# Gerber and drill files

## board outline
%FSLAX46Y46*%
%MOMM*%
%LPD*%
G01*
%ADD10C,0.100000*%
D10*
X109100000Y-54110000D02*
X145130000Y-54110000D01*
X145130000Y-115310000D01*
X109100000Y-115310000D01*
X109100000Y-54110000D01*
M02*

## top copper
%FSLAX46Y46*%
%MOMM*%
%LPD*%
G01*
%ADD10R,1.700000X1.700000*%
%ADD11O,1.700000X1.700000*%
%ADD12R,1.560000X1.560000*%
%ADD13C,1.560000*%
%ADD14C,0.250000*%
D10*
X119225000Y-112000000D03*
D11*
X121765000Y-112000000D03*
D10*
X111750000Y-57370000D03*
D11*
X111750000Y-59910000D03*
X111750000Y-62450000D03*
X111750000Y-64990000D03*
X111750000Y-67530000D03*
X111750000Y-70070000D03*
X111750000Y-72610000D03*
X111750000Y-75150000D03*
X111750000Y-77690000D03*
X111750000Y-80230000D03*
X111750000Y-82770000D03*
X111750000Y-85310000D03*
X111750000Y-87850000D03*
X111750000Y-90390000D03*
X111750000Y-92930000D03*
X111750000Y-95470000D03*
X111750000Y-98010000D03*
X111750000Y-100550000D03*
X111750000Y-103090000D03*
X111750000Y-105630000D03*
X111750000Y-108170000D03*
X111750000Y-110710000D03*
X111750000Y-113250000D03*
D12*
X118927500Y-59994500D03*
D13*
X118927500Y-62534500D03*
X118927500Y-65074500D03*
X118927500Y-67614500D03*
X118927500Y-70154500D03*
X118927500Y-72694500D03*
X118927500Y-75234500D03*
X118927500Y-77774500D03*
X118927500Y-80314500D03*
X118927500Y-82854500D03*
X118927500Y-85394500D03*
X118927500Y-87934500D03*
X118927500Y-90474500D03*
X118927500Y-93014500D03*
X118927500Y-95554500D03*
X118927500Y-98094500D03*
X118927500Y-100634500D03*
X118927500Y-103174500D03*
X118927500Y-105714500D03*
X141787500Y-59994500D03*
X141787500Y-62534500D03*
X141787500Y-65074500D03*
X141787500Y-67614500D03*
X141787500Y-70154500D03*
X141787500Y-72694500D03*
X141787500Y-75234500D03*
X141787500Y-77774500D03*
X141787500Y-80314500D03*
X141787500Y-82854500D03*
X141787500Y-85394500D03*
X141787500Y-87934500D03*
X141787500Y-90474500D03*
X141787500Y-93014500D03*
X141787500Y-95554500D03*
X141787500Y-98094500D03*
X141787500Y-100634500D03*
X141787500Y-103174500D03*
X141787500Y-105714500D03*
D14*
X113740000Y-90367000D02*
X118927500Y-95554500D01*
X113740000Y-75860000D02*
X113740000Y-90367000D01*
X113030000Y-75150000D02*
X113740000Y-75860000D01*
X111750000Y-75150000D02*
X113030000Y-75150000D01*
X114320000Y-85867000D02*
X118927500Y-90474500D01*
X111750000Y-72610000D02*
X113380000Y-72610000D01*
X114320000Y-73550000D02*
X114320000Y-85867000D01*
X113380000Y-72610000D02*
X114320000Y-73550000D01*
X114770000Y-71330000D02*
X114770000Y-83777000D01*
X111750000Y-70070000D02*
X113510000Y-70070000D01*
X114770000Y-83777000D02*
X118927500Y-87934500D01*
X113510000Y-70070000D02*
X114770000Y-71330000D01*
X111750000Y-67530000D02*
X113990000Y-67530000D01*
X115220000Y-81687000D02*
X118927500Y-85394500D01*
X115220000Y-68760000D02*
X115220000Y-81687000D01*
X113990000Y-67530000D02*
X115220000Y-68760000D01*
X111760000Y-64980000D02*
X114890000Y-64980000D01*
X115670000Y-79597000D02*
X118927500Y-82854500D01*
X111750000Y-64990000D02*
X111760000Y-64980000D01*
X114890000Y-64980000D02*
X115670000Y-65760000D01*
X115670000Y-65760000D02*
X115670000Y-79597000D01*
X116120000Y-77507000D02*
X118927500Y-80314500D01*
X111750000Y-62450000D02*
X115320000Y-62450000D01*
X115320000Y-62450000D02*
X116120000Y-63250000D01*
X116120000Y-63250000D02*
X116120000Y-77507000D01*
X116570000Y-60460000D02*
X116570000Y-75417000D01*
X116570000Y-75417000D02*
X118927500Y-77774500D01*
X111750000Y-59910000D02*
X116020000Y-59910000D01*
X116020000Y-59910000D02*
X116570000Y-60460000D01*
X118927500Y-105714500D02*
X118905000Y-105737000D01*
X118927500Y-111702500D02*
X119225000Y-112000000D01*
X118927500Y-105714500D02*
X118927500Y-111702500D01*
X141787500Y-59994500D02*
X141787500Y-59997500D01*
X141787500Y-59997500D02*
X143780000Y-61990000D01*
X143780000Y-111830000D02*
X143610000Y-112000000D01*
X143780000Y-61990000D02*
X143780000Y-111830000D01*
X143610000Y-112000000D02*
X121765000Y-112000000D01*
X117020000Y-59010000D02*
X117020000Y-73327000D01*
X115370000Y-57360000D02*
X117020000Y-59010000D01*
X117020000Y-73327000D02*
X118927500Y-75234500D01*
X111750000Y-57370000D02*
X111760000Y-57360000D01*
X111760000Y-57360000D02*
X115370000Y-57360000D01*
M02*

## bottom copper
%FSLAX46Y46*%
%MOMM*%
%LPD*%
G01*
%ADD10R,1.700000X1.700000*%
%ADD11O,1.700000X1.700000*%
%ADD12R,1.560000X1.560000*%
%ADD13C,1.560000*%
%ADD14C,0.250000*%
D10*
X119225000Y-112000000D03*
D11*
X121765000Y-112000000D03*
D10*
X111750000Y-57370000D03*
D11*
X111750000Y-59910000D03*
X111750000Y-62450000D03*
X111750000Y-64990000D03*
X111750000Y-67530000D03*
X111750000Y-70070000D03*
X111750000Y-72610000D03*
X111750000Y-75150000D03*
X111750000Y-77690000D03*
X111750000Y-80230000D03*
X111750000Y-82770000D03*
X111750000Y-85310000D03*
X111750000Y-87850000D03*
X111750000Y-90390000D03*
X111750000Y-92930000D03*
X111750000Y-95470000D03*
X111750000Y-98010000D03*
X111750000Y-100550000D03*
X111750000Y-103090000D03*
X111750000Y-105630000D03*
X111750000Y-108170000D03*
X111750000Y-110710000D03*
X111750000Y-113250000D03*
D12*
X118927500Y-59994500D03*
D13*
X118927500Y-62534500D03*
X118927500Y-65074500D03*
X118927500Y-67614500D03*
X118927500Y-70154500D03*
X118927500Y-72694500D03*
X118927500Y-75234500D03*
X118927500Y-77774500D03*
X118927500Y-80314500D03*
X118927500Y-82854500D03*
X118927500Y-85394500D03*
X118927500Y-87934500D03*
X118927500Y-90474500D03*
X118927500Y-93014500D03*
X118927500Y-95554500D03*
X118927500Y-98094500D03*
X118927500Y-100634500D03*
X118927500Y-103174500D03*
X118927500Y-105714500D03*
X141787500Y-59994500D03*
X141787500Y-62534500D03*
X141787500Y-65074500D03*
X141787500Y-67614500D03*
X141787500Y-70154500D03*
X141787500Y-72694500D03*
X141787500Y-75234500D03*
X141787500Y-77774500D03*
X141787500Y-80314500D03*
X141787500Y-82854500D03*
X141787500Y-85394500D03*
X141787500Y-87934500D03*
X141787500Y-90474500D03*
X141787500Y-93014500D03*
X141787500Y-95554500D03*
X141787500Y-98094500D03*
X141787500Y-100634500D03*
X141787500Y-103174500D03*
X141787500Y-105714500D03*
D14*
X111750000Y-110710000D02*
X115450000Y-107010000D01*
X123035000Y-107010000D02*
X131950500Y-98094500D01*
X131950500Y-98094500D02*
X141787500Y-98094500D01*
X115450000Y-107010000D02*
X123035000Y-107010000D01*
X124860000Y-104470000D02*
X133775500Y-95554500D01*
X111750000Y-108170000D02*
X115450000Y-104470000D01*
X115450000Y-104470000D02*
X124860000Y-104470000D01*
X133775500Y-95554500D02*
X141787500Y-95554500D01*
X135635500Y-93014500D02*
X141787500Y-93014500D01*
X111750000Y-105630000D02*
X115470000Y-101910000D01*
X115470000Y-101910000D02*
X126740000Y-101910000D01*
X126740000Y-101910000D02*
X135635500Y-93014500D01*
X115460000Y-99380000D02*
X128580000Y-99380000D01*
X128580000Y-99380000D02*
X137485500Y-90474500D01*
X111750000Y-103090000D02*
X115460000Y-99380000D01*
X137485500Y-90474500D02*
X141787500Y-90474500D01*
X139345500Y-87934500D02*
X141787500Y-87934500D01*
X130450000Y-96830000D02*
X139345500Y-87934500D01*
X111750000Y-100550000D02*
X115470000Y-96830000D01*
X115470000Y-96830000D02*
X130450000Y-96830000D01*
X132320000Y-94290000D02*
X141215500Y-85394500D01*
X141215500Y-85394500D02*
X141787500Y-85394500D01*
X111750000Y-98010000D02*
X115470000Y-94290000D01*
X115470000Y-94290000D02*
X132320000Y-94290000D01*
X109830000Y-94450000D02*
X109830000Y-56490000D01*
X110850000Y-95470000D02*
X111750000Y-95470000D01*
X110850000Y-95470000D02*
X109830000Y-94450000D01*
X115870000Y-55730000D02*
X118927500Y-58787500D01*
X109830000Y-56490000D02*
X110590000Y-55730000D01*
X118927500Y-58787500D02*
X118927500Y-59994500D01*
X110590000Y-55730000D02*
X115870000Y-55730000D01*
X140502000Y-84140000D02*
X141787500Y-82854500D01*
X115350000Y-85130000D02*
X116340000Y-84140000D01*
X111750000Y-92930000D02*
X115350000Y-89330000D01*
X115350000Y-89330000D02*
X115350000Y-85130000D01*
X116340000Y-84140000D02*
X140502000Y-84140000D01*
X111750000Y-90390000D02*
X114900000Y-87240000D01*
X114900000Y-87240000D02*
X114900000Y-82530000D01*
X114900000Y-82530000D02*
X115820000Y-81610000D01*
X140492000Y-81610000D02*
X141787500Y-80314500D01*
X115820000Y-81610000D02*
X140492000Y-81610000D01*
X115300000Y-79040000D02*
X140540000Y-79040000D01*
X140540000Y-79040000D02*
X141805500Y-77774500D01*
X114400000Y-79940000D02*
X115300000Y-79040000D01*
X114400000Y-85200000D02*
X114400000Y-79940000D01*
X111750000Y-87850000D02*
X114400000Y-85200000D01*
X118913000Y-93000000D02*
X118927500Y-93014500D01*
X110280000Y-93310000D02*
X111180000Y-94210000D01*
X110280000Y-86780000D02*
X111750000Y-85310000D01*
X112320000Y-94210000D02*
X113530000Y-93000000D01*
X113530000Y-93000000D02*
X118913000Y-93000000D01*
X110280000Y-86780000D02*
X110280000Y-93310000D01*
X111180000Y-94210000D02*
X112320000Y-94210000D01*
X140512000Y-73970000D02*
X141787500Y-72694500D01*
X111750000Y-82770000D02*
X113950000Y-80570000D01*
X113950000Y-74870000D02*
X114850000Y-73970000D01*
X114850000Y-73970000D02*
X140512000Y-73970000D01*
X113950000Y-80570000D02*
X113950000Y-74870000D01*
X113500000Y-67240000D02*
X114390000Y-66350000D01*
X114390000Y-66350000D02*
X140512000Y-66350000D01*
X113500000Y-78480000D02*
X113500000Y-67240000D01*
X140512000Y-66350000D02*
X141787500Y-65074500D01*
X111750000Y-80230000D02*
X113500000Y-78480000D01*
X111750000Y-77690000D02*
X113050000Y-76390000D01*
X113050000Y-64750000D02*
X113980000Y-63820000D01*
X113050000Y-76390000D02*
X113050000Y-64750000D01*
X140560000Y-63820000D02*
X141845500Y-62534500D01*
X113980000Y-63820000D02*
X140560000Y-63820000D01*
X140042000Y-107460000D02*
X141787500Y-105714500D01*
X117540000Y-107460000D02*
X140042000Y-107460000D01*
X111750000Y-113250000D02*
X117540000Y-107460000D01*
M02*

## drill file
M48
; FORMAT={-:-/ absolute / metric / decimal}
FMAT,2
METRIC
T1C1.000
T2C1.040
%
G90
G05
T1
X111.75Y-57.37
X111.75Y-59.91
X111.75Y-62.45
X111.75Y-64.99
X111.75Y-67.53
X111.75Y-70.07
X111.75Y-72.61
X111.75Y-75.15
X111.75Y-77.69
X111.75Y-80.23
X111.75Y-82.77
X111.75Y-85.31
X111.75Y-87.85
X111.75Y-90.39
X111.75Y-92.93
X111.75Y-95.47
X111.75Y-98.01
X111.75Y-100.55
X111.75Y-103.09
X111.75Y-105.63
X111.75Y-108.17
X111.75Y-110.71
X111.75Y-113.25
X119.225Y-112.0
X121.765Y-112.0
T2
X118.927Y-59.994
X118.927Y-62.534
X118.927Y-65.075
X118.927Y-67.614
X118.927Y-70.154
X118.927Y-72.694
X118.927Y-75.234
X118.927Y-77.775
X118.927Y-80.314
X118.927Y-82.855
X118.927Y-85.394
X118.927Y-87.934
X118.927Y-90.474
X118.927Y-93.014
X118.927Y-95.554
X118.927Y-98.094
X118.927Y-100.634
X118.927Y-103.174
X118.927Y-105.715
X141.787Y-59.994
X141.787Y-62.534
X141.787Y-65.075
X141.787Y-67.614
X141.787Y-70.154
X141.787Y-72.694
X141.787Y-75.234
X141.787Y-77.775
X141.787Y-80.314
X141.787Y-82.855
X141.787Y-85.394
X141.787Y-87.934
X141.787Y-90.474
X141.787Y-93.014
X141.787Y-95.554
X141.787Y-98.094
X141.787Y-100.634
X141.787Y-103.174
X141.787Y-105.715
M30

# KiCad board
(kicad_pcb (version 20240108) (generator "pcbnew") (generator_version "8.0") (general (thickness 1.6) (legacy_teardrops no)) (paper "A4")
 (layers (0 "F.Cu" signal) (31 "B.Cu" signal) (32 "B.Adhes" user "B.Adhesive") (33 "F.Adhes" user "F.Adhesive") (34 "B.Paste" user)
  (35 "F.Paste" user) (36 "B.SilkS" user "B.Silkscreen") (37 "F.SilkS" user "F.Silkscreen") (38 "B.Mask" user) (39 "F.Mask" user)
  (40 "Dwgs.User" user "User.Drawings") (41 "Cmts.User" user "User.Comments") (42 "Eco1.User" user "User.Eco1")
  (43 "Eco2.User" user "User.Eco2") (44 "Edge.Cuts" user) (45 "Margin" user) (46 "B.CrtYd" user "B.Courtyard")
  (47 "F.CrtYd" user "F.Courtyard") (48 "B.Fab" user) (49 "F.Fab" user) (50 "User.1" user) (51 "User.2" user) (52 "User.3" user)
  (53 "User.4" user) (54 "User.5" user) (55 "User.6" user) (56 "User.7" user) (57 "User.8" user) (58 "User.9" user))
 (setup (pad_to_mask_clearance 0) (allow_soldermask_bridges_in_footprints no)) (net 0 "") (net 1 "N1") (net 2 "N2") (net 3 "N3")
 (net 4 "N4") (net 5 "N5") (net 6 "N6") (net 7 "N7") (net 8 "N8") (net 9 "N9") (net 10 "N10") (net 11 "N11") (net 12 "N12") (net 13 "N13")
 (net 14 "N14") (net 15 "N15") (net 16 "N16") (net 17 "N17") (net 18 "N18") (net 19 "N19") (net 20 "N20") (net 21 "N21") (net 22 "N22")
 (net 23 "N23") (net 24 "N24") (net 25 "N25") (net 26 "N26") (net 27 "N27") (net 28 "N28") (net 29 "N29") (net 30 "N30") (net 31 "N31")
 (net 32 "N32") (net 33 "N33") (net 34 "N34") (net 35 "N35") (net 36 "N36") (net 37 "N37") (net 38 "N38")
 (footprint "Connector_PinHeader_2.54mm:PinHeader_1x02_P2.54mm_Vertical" (layer "F.Cu") (at 119.225 112 90)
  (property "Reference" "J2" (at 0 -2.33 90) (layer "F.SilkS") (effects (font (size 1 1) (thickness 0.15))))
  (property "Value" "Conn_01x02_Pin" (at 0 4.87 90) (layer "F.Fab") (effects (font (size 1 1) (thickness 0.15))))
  (pad "1" thru_hole rect (at 0 0 90) (size 1.7 1.7) (drill 1) (layers "*.Cu" "*.Mask") (remove_unused_layers no) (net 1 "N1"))
  (pad "2" thru_hole oval (at 0 2.54 90) (size 1.7 1.7) (drill 1) (layers "*.Cu" "*.Mask") (remove_unused_layers no) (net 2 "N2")))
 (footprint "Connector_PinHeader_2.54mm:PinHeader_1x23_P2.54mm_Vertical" (layer "F.Cu") (at 111.75 57.37)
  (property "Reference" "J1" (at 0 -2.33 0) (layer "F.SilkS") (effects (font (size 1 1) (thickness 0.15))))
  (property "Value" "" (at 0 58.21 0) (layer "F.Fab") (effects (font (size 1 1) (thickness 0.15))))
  (pad "1" thru_hole rect (at 0 0) (size 1.7 1.7) (drill 1) (layers "*.Cu" "*.Mask") (remove_unused_layers no) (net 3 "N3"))
  (pad "2" thru_hole oval (at 0 2.54) (size 1.7 1.7) (drill 1) (layers "*.Cu" "*.Mask") (remove_unused_layers no) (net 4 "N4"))
  (pad "3" thru_hole oval (at 0 5.08) (size 1.7 1.7) (drill 1) (layers "*.Cu" "*.Mask") (remove_unused_layers no) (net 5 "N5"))
  (pad "4" thru_hole oval (at 0 7.62) (size 1.7 1.7) (drill 1) (layers "*.Cu" "*.Mask") (remove_unused_layers no) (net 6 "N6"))
  (pad "5" thru_hole oval (at 0 10.16) (size 1.7 1.7) (drill 1) (layers "*.Cu" "*.Mask") (remove_unused_layers no) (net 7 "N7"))
  (pad "6" thru_hole oval (at 0 12.7) (size 1.7 1.7) (drill 1) (layers "*.Cu" "*.Mask") (remove_unused_layers no) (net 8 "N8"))
  (pad "7" thru_hole oval (at 0 15.24) (size 1.7 1.7) (drill 1) (layers "*.Cu" "*.Mask") (remove_unused_layers no) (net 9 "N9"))
  (pad "8" thru_hole oval (at 0 17.78) (size 1.7 1.7) (drill 1) (layers "*.Cu" "*.Mask") (remove_unused_layers no) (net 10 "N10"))
  (pad "9" thru_hole oval (at 0 20.32) (size 1.7 1.7) (drill 1) (layers "*.Cu" "*.Mask") (remove_unused_layers no) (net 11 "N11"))
  (pad "10" thru_hole oval (at 0 22.86) (size 1.7 1.7) (drill 1) (layers "*.Cu" "*.Mask") (remove_unused_layers no) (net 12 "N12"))
  (pad "11" thru_hole oval (at 0 25.4) (size 1.7 1.7) (drill 1) (layers "*.Cu" "*.Mask") (remove_unused_layers no) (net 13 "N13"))
  (pad "12" thru_hole oval (at 0 27.94) (size 1.7 1.7) (drill 1) (layers "*.Cu" "*.Mask") (remove_unused_layers no) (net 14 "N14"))
  (pad "13" thru_hole oval (at 0 30.48) (size 1.7 1.7) (drill 1) (layers "*.Cu" "*.Mask") (remove_unused_layers no) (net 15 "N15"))
  (pad "14" thru_hole oval (at 0 33.02) (size 1.7 1.7) (drill 1) (layers "*.Cu" "*.Mask") (remove_unused_layers no) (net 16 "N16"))
  (pad "15" thru_hole oval (at 0 35.56) (size 1.7 1.7) (drill 1) (layers "*.Cu" "*.Mask") (remove_unused_layers no) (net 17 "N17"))
  (pad "16" thru_hole oval (at 0 38.1) (size 1.7 1.7) (drill 1) (layers "*.Cu" "*.Mask") (remove_unused_layers no) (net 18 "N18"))
  (pad "17" thru_hole oval (at 0 40.64) (size 1.7 1.7) (drill 1) (layers "*.Cu" "*.Mask") (remove_unused_layers no) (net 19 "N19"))
  (pad "18" thru_hole oval (at 0 43.18) (size 1.7 1.7) (drill 1) (layers "*.Cu" "*.Mask") (remove_unused_layers no) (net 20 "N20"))
  (pad "19" thru_hole oval (at 0 45.72) (size 1.7 1.7) (drill 1) (layers "*.Cu" "*.Mask") (remove_unused_layers no) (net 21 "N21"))
  (pad "20" thru_hole oval (at 0 48.26) (size 1.7 1.7) (drill 1) (layers "*.Cu" "*.Mask") (remove_unused_layers no) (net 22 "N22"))
  (pad "21" thru_hole oval (at 0 50.8) (size 1.7 1.7) (drill 1) (layers "*.Cu" "*.Mask") (remove_unused_layers no) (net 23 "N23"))
  (pad "22" thru_hole oval (at 0 53.34) (size 1.7 1.7) (drill 1) (layers "*.Cu" "*.Mask") (remove_unused_layers no) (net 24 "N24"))
  (pad "23" thru_hole oval (at 0 55.88) (size 1.7 1.7) (drill 1) (layers "*.Cu" "*.Mask") (remove_unused_layers no) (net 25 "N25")))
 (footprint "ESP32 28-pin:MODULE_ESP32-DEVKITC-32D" (layer "F.Cu") (at 131.6275 79.7545)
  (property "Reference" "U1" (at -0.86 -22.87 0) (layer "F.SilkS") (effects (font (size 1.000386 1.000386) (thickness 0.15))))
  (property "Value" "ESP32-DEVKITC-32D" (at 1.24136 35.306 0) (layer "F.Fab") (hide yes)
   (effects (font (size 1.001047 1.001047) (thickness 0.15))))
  (pad "J2-1" thru_hole rect (at -12.7 -19.76) (size 1.56 1.56) (drill 1.04) (layers "*.Cu" "*.Mask") (remove_unused_layers no)
   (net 18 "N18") (solder_mask_margin 0.102))
  (pad "J2-2" thru_hole circle (at -12.7 -17.22) (size 1.56 1.56) (drill 1.04) (layers "*.Cu" "*.Mask") (remove_unused_layers no)
   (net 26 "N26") (solder_mask_margin 0.102))
  (pad "J2-3" thru_hole circle (at -12.7 -14.68) (size 1.56 1.56) (drill 1.04) (layers "*.Cu" "*.Mask") (remove_unused_layers no)
   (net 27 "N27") (solder_mask_margin 0.102))
  (pad "J2-4" thru_hole circle (at -12.7 -12.14) (size 1.56 1.56) (drill 1.04) (layers "*.Cu" "*.Mask") (remove_unused_layers no)
   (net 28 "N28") (solder_mask_margin 0.102))
  (pad "J2-5" thru_hole circle (at -12.7 -9.6) (size 1.56 1.56) (drill 1.04) (layers "*.Cu" "*.Mask") (remove_unused_layers no)
   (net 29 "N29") (solder_mask_margin 0.102))
  (pad "J2-6" thru_hole circle (at -12.7 -7.06) (size 1.56 1.56) (drill 1.04) (layers "*.Cu" "*.Mask") (remove_unused_layers no)
   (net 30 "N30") (solder_mask_margin 0.102))
  (pad "J2-7" thru_hole circle (at -12.7 -4.52) (size 1.56 1.56) (drill 1.04) (layers "*.Cu" "*.Mask") (remove_unused_layers no)
   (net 3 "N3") (solder_mask_margin 0.102))
  (pad "J2-8" thru_hole circle (at -12.7 -1.98) (size 1.56 1.56) (drill 1.04) (layers "*.Cu" "*.Mask") (remove_unused_layers no)
   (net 4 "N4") (solder_mask_margin 0.102))
  (pad "J2-9" thru_hole circle (at -12.7 0.56) (size 1.56 1.56) (drill 1.04) (layers "*.Cu" "*.Mask") (remove_unused_layers no) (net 5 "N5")
   (solder_mask_margin 0.102))
  (pad "J2-10" thru_hole circle (at -12.7 3.1) (size 1.56 1.56) (drill 1.04) (layers "*.Cu" "*.Mask") (remove_unused_layers no) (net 6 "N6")
   (solder_mask_margin 0.102))
  (pad "J2-11" thru_hole circle (at -12.7 5.64) (size 1.56 1.56) (drill 1.04) (layers "*.Cu" "*.Mask") (remove_unused_layers no)
   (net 7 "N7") (solder_mask_margin 0.102))
  (pad "J2-12" thru_hole circle (at -12.7 8.18) (size 1.56 1.56) (drill 1.04) (layers "*.Cu" "*.Mask") (remove_unused_layers no)
   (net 8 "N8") (solder_mask_margin 0.102))
  (pad "J2-13" thru_hole circle (at -12.7 10.72) (size 1.56 1.56) (drill 1.04) (layers "*.Cu" "*.Mask") (remove_unused_layers no)
   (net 9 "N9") (solder_mask_margin 0.102))
  (pad "J2-14" thru_hole circle (at -12.7 13.26) (size 1.56 1.56) (drill 1.04) (layers "*.Cu" "*.Mask") (remove_unused_layers no)
   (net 14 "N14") (solder_mask_margin 0.102))
  (pad "J2-15" thru_hole circle (at -12.7 15.8) (size 1.56 1.56) (drill 1.04) (layers "*.Cu" "*.Mask") (remove_unused_layers no)
   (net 10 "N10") (solder_mask_margin 0.102))
  (pad "J2-16" thru_hole circle (at -12.7 18.34) (size 1.56 1.56) (drill 1.04) (layers "*.Cu" "*.Mask") (remove_unused_layers no)
   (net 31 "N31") (solder_mask_margin 0.102))
  (pad "J2-17" thru_hole circle (at -12.7 20.88) (size 1.56 1.56) (drill 1.04) (layers "*.Cu" "*.Mask") (remove_unused_layers no)
   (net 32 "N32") (solder_mask_margin 0.102))
  (pad "J2-18" thru_hole circle (at -12.7 23.42) (size 1.56 1.56) (drill 1.04) (layers "*.Cu" "*.Mask") (remove_unused_layers no)
   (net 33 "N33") (solder_mask_margin 0.102))
  (pad "J2-19" thru_hole circle (at -12.7 25.96) (size 1.56 1.56) (drill 1.04) (layers "*.Cu" "*.Mask") (remove_unused_layers no)
   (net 1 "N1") (solder_mask_margin 0.102))
  (pad "J3-1" thru_hole circle (at 10.16 -19.76) (size 1.56 1.56) (drill 1.04) (layers "*.Cu" "*.Mask") (remove_unused_layers no)
   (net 2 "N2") (solder_mask_margin 0.102))
  (pad "J3-2" thru_hole circle (at 10.16 -17.22) (size 1.56 1.56) (drill 1.04) (layers "*.Cu" "*.Mask") (remove_unused_layers no)
   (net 11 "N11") (solder_mask_margin 0.102))
  (pad "J3-3" thru_hole circle (at 10.16 -14.68) (size 1.56 1.56) (drill 1.04) (layers "*.Cu" "*.Mask") (remove_unused_layers no)
   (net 12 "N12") (solder_mask_margin 0.102))
  (pad "J3-4" thru_hole circle (at 10.16 -12.14) (size 1.56 1.56) (drill 1.04) (layers "*.Cu" "*.Mask") (remove_unused_layers no)
   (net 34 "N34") (solder_mask_margin 0.102))
  (pad "J3-5" thru_hole circle (at 10.16 -9.6) (size 1.56 1.56) (drill 1.04) (layers "*.Cu" "*.Mask") (remove_unused_layers no)
   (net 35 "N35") (solder_mask_margin 0.102))
  (pad "J3-6" thru_hole circle (at 10.16 -7.06) (size 1.56 1.56) (drill 1.04) (layers "*.Cu" "*.Mask") (remove_unused_layers no)
   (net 13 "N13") (solder_mask_margin 0.102))
  (pad "J3-7" thru_hole circle (at 10.16 -4.52) (size 1.56 1.56) (drill 1.04) (layers "*.Cu" "*.Mask") (remove_unused_layers no)
   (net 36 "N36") (solder_mask_margin 0.102))
  (pad "J3-8" thru_hole circle (at 10.16 -1.98) (size 1.56 1.56) (drill 1.04) (layers "*.Cu" "*.Mask") (remove_unused_layers no)
   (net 15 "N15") (solder_mask_margin 0.102))
  (pad "J3-9" thru_hole circle (at 10.16 0.56) (size 1.56 1.56) (drill 1.04) (layers "*.Cu" "*.Mask") (remove_unused_layers no)
   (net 16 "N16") (solder_mask_margin 0.102))
  (pad "J3-10" thru_hole circle (at 10.16 3.1) (size 1.56 1.56) (drill 1.04) (layers "*.Cu" "*.Mask") (remove_unused_layers no)
   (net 17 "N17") (solder_mask_margin 0.102))
  (pad "J3-11" thru_hole circle (at 10.16 5.64) (size 1.56 1.56) (drill 1.04) (layers "*.Cu" "*.Mask") (remove_unused_layers no)
   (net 19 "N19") (solder_mask_margin 0.102))
  (pad "J3-12" thru_hole circle (at 10.16 8.18) (size 1.56 1.56) (drill 1.04) (layers "*.Cu" "*.Mask") (remove_unused_layers no)
   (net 20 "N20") (solder_mask_margin 0.102))
  (pad "J3-13" thru_hole circle (at 10.16 10.72) (size 1.56 1.56) (drill 1.04) (layers "*.Cu" "*.Mask") (remove_unused_layers no)
   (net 21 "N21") (solder_mask_margin 0.102))
  (pad "J3-14" thru_hole circle (at 10.16 13.26) (size 1.56 1.56) (drill 1.04) (layers "*.Cu" "*.Mask") (remove_unused_layers no)
   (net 22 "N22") (solder_mask_margin 0.102))
  (pad "J3-15" thru_hole circle (at 10.16 15.8) (size 1.56 1.56) (drill 1.04) (layers "*.Cu" "*.Mask") (remove_unused_layers no)
   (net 23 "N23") (solder_mask_margin 0.102))
  (pad "J3-16" thru_hole circle (at 10.16 18.34) (size 1.56 1.56) (drill 1.04) (layers "*.Cu" "*.Mask") (remove_unused_layers no)
   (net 24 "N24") (solder_mask_margin 0.102))
  (pad "J3-17" thru_hole circle (at 10.16 20.88) (size 1.56 1.56) (drill 1.04) (layers "*.Cu" "*.Mask") (remove_unused_layers no)
   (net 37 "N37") (solder_mask_margin 0.102))
  (pad "J3-18" thru_hole circle (at 10.16 23.42) (size 1.56 1.56) (drill 1.04) (layers "*.Cu" "*.Mask") (remove_unused_layers no)
   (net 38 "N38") (solder_mask_margin 0.102))
  (pad "J3-19" thru_hole circle (at 10.16 25.96) (size 1.56 1.56) (drill 1.04) (layers "*.Cu" "*.Mask") (remove_unused_layers no)
   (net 25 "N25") (solder_mask_margin 0.102)))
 (gr_rect (start 109.1 54.11) (end 145.13 115.31) (stroke (width 0.1) (type default)) (fill none) (layer "Edge.Cuts"))
 (segment (start 111.75 110.71) (end 115.45 107.01) (width 0.25) (layer "B.Cu") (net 24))
 (segment (start 123.035 107.01) (end 131.9505 98.0945) (width 0.25) (layer "B.Cu") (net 24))
 (segment (start 131.9505 98.0945) (end 141.7875 98.0945) (width 0.25) (layer "B.Cu") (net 24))
 (segment (start 115.45 107.01) (end 123.035 107.01) (width 0.25) (layer "B.Cu") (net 24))
 (segment (start 124.86 104.47) (end 133.7755 95.5545) (width 0.25) (layer "B.Cu") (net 23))
 (segment (start 111.75 108.17) (end 115.45 104.47) (width 0.25) (layer "B.Cu") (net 23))
 (segment (start 115.45 104.47) (end 124.86 104.47) (width 0.25) (layer "B.Cu") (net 23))
 (segment (start 133.7755 95.5545) (end 141.7875 95.5545) (width 0.25) (layer "B.Cu") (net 23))
 (segment (start 135.6355 93.0145) (end 141.7875 93.0145) (width 0.25) (layer "B.Cu") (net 22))
 (segment (start 111.75 105.63) (end 115.47 101.91) (width 0.25) (layer "B.Cu") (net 22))
 (segment (start 115.47 101.91) (end 126.74 101.91) (width 0.25) (layer "B.Cu") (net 22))
 (segment (start 126.74 101.91) (end 135.6355 93.0145) (width 0.25) (layer "B.Cu") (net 22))
 (segment (start 115.46 99.38) (end 128.58 99.38) (width 0.25) (layer "B.Cu") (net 21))
 (segment (start 128.58 99.38) (end 137.4855 90.4745) (width 0.25) (layer "B.Cu") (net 21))
 (segment (start 111.75 103.09) (end 115.46 99.38) (width 0.25) (layer "B.Cu") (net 21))
 (segment (start 137.4855 90.4745) (end 141.7875 90.4745) (width 0.25) (layer "B.Cu") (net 21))
 (segment (start 139.3455 87.9345) (end 141.7875 87.9345) (width 0.25) (layer "B.Cu") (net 20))
 (segment (start 130.45 96.83) (end 139.3455 87.9345) (width 0.25) (layer "B.Cu") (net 20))
 (segment (start 111.75 100.55) (end 115.47 96.83) (width 0.25) (layer "B.Cu") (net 20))
 (segment (start 115.47 96.83) (end 130.45 96.83) (width 0.25) (layer "B.Cu") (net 20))
 (segment (start 132.32 94.29) (end 141.2155 85.3945) (width 0.25) (layer "B.Cu") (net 19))
 (segment (start 141.2155 85.3945) (end 141.7875 85.3945) (width 0.25) (layer "B.Cu") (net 19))
 (segment (start 111.75 98.01) (end 115.47 94.29) (width 0.25) (layer "B.Cu") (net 19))
 (segment (start 115.47 94.29) (end 132.32 94.29) (width 0.25) (layer "B.Cu") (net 19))
 (segment (start 109.83 94.45) (end 109.83 56.49) (width 0.25) (layer "B.Cu") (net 18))
 (segment (start 110.85 95.47) (end 111.75 95.47) (width 0.25) (layer "B.Cu") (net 18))
 (segment (start 110.85 95.47) (end 109.83 94.45) (width 0.25) (layer "B.Cu") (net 18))
 (segment (start 115.87 55.73) (end 118.9275 58.7875) (width 0.25) (layer "B.Cu") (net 18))
 (segment (start 109.83 56.49) (end 110.59 55.73) (width 0.25) (layer "B.Cu") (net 18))
 (segment (start 118.9275 58.7875) (end 118.9275 59.9945) (width 0.25) (layer "B.Cu") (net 18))
 (segment (start 110.59 55.73) (end 115.87 55.73) (width 0.25) (layer "B.Cu") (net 18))
 (segment (start 140.502 84.14) (end 141.7875 82.8545) (width 0.25) (layer "B.Cu") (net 17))
 (segment (start 115.35 85.13) (end 116.34 84.14) (width 0.25) (layer "B.Cu") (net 17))
 (segment (start 111.75 92.93) (end 115.35 89.33) (width 0.25) (layer "B.Cu") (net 17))
 (segment (start 115.35 89.33) (end 115.35 85.13) (width 0.25) (layer "B.Cu") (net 17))
 (segment (start 116.34 84.14) (end 140.502 84.14) (width 0.25) (layer "B.Cu") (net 17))
 (segment (start 111.75 90.39) (end 114.9 87.24) (width 0.25) (layer "B.Cu") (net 16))
 (segment (start 114.9 87.24) (end 114.9 82.53) (width 0.25) (layer "B.Cu") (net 16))
 (segment (start 114.9 82.53) (end 115.82 81.61) (width 0.25) (layer "B.Cu") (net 16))
 (segment (start 140.492 81.61) (end 141.7875 80.3145) (width 0.25) (layer "B.Cu") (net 16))
 (segment (start 115.82 81.61) (end 140.492 81.61) (width 0.25) (layer "B.Cu") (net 16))
 (segment (start 115.3 79.04) (end 140.54 79.04) (width 0.25) (layer "B.Cu") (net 15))
 (segment (start 140.54 79.04) (end 141.8055 77.7745) (width 0.25) (layer "B.Cu") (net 15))
 (segment (start 114.4 79.94) (end 115.3 79.04) (width 0.25) (layer "B.Cu") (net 15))
 (segment (start 114.4 85.2) (end 114.4 79.94) (width 0.25) (layer "B.Cu") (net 15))
 (segment (start 111.75 87.85) (end 114.4 85.2) (width 0.25) (layer "B.Cu") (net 15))
 (segment (start 118.913 93) (end 118.9275 93.0145) (width 0.25) (layer "B.Cu") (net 14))
 (segment (start 110.28 93.31) (end 111.18 94.21) (width 0.25) (layer "B.Cu") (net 14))
 (segment (start 110.28 86.78) (end 111.75 85.31) (width 0.25) (layer "B.Cu") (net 14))
 (segment (start 112.32 94.21) (end 113.53 93) (width 0.25) (layer "B.Cu") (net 14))
 (segment (start 113.53 93) (end 118.913 93) (width 0.25) (layer "B.Cu") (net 14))
 (segment (start 110.28 86.78) (end 110.28 93.31) (width 0.25) (layer "B.Cu") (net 14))
 (segment (start 111.18 94.21) (end 112.32 94.21) (width 0.25) (layer "B.Cu") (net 14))
 (segment (start 140.512 73.97) (end 141.7875 72.6945) (width 0.25) (layer "B.Cu") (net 13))
 (segment (start 111.75 82.77) (end 113.95 80.57) (width 0.25) (layer "B.Cu") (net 13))
 (segment (start 113.95 74.87) (end 114.85 73.97) (width 0.25) (layer "B.Cu") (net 13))
 (segment (start 114.85 73.97) (end 140.512 73.97) (width 0.25) (layer "B.Cu") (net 13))
 (segment (start 113.95 80.57) (end 113.95 74.87) (width 0.25) (layer "B.Cu") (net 13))
 (segment (start 113.5 67.24) (end 114.39 66.35) (width 0.25) (layer "B.Cu") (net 12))
 (segment (start 114.39 66.35) (end 140.512 66.35) (width 0.25) (layer "B.Cu") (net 12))
 (segment (start 113.5 78.48) (end 113.5 67.24) (width 0.25) (layer "B.Cu") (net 12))
 (segment (start 140.512 66.35) (end 141.7875 65.0745) (width 0.25) (layer "B.Cu") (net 12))
 (segment (start 111.75 80.23) (end 113.5 78.48) (width 0.25) (layer "B.Cu") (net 12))
 (segment (start 111.75 77.69) (end 113.05 76.39) (width 0.25) (layer "B.Cu") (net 11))
 (segment (start 113.05 64.75) (end 113.98 63.82) (width 0.25) (layer "B.Cu") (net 11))
 (segment (start 113.05 76.39) (end 113.05 64.75) (width 0.25) (layer "B.Cu") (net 11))
 (segment (start 140.56 63.82) (end 141.8455 62.5345) (width 0.25) (layer "B.Cu") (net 11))
 (segment (start 113.98 63.82) (end 140.56 63.82) (width 0.25) (layer "B.Cu") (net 11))
 (segment (start 113.74 90.367) (end 118.9275 95.5545) (width 0.25) (layer "F.Cu") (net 10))
 (segment (start 113.74 75.86) (end 113.74 90.367) (width 0.25) (layer "F.Cu") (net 10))
 (segment (start 113.03 75.15) (end 113.74 75.86) (width 0.25) (layer "F.Cu") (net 10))
 (segment (start 111.75 75.15) (end 113.03 75.15) (width 0.25) (layer "F.Cu") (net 10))
 (segment (start 114.32 85.867) (end 118.9275 90.4745) (width 0.25) (layer "F.Cu") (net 9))
 (segment (start 111.75 72.61) (end 113.38 72.61) (width 0.25) (layer "F.Cu") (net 9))
 (segment (start 114.32 73.55) (end 114.32 85.867) (width 0.25) (layer "F.Cu") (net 9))
 (segment (start 113.38 72.61) (end 114.32 73.55) (width 0.25) (layer "F.Cu") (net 9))
 (segment (start 114.77 71.33) (end 114.77 83.777) (width 0.25) (layer "F.Cu") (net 8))
 (segment (start 111.75 70.07) (end 113.51 70.07) (width 0.25) (layer "F.Cu") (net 8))
 (segment (start 114.77 83.777) (end 118.9275 87.9345) (width 0.25) (layer "F.Cu") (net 8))
 (segment (start 113.51 70.07) (end 114.77 71.33) (width 0.25) (layer "F.Cu") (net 8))
 (segment (start 111.75 67.53) (end 113.99 67.53) (width 0.25) (layer "F.Cu") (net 7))
 (segment (start 115.22 81.687) (end 118.9275 85.3945) (width 0.25) (layer "F.Cu") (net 7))
 (segment (start 115.22 68.76) (end 115.22 81.687) (width 0.25) (layer "F.Cu") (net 7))
 (segment (start 113.99 67.53) (end 115.22 68.76) (width 0.25) (layer "F.Cu") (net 7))
 (segment (start 111.76 64.98) (end 114.89 64.98) (width 0.25) (layer "F.Cu") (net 6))
 (segment (start 115.67 79.597) (end 118.9275 82.8545) (width 0.25) (layer "F.Cu") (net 6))
 (segment (start 111.75 64.99) (end 111.76 64.98) (width 0.25) (layer "F.Cu") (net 6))
 (segment (start 114.89 64.98) (end 115.67 65.76) (width 0.25) (layer "F.Cu") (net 6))
 (segment (start 115.67 65.76) (end 115.67 79.597) (width 0.25) (layer "F.Cu") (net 6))
 (segment (start 116.12 77.507) (end 118.9275 80.3145) (width 0.25) (layer "F.Cu") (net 5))
 (segment (start 111.75 62.45) (end 115.32 62.45) (width 0.25) (layer "F.Cu") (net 5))
 (segment (start 115.32 62.45) (end 116.12 63.25) (width 0.25) (layer "F.Cu") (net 5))
 (segment (start 116.12 63.25) (end 116.12 77.507) (width 0.25) (layer "F.Cu") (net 5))
 (segment (start 116.57 60.46) (end 116.57 75.417) (width 0.25) (layer "F.Cu") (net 4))
 (segment (start 116.57 75.417) (end 118.9275 77.7745) (width 0.25) (layer "F.Cu") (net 4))
 (segment (start 111.75 59.91) (end 116.02 59.91) (width 0.25) (layer "F.Cu") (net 4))
 (segment (start 116.02 59.91) (end 116.57 60.46) (width 0.25) (layer "F.Cu") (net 4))
 (segment (start 118.9275 105.7145) (end 118.905 105.737) (width 0.25) (layer "F.Cu") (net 1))
 (segment (start 118.9275 111.7025) (end 119.225 112) (width 0.25) (layer "F.Cu") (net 1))
 (segment (start 118.9275 105.7145) (end 118.9275 111.7025) (width 0.25) (layer "F.Cu") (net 1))
 (segment (start 141.7875 59.9945) (end 141.7875 59.9975) (width 0.25) (layer "F.Cu") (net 2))
 (segment (start 141.7875 59.9975) (end 143.78 61.99) (width 0.25) (layer "F.Cu") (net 2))
 (segment (start 143.78 111.83) (end 143.61 112) (width 0.25) (layer "F.Cu") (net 2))
 (segment (start 143.78 61.99) (end 143.78 111.83) (width 0.25) (layer "F.Cu") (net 2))
 (segment (start 143.61 112) (end 121.765 112) (width 0.25) (layer "F.Cu") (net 2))
 (segment (start 117.02 59.01) (end 117.02 73.327) (width 0.25) (layer "F.Cu") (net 3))
 (segment (start 115.37 57.36) (end 117.02 59.01) (width 0.25) (layer "F.Cu") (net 3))
 (segment (start 117.02 73.327) (end 118.9275 75.2345) (width 0.25) (layer "F.Cu") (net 3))
 (segment (start 111.75 57.37) (end 111.76 57.36) (width 0.25) (layer "F.Cu") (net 3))
 (segment (start 111.76 57.36) (end 115.37 57.36) (width 0.25) (layer "F.Cu") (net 3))
 (segment (start 140.042 107.46) (end 141.7875 105.7145) (width 0.25) (layer "B.Cu") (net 25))
 (segment (start 117.54 107.46) (end 140.042 107.46) (width 0.25) (layer "B.Cu") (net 25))
 (segment (start 111.75 113.25) (end 117.54 107.46) (width 0.25) (layer "B.Cu") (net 25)))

